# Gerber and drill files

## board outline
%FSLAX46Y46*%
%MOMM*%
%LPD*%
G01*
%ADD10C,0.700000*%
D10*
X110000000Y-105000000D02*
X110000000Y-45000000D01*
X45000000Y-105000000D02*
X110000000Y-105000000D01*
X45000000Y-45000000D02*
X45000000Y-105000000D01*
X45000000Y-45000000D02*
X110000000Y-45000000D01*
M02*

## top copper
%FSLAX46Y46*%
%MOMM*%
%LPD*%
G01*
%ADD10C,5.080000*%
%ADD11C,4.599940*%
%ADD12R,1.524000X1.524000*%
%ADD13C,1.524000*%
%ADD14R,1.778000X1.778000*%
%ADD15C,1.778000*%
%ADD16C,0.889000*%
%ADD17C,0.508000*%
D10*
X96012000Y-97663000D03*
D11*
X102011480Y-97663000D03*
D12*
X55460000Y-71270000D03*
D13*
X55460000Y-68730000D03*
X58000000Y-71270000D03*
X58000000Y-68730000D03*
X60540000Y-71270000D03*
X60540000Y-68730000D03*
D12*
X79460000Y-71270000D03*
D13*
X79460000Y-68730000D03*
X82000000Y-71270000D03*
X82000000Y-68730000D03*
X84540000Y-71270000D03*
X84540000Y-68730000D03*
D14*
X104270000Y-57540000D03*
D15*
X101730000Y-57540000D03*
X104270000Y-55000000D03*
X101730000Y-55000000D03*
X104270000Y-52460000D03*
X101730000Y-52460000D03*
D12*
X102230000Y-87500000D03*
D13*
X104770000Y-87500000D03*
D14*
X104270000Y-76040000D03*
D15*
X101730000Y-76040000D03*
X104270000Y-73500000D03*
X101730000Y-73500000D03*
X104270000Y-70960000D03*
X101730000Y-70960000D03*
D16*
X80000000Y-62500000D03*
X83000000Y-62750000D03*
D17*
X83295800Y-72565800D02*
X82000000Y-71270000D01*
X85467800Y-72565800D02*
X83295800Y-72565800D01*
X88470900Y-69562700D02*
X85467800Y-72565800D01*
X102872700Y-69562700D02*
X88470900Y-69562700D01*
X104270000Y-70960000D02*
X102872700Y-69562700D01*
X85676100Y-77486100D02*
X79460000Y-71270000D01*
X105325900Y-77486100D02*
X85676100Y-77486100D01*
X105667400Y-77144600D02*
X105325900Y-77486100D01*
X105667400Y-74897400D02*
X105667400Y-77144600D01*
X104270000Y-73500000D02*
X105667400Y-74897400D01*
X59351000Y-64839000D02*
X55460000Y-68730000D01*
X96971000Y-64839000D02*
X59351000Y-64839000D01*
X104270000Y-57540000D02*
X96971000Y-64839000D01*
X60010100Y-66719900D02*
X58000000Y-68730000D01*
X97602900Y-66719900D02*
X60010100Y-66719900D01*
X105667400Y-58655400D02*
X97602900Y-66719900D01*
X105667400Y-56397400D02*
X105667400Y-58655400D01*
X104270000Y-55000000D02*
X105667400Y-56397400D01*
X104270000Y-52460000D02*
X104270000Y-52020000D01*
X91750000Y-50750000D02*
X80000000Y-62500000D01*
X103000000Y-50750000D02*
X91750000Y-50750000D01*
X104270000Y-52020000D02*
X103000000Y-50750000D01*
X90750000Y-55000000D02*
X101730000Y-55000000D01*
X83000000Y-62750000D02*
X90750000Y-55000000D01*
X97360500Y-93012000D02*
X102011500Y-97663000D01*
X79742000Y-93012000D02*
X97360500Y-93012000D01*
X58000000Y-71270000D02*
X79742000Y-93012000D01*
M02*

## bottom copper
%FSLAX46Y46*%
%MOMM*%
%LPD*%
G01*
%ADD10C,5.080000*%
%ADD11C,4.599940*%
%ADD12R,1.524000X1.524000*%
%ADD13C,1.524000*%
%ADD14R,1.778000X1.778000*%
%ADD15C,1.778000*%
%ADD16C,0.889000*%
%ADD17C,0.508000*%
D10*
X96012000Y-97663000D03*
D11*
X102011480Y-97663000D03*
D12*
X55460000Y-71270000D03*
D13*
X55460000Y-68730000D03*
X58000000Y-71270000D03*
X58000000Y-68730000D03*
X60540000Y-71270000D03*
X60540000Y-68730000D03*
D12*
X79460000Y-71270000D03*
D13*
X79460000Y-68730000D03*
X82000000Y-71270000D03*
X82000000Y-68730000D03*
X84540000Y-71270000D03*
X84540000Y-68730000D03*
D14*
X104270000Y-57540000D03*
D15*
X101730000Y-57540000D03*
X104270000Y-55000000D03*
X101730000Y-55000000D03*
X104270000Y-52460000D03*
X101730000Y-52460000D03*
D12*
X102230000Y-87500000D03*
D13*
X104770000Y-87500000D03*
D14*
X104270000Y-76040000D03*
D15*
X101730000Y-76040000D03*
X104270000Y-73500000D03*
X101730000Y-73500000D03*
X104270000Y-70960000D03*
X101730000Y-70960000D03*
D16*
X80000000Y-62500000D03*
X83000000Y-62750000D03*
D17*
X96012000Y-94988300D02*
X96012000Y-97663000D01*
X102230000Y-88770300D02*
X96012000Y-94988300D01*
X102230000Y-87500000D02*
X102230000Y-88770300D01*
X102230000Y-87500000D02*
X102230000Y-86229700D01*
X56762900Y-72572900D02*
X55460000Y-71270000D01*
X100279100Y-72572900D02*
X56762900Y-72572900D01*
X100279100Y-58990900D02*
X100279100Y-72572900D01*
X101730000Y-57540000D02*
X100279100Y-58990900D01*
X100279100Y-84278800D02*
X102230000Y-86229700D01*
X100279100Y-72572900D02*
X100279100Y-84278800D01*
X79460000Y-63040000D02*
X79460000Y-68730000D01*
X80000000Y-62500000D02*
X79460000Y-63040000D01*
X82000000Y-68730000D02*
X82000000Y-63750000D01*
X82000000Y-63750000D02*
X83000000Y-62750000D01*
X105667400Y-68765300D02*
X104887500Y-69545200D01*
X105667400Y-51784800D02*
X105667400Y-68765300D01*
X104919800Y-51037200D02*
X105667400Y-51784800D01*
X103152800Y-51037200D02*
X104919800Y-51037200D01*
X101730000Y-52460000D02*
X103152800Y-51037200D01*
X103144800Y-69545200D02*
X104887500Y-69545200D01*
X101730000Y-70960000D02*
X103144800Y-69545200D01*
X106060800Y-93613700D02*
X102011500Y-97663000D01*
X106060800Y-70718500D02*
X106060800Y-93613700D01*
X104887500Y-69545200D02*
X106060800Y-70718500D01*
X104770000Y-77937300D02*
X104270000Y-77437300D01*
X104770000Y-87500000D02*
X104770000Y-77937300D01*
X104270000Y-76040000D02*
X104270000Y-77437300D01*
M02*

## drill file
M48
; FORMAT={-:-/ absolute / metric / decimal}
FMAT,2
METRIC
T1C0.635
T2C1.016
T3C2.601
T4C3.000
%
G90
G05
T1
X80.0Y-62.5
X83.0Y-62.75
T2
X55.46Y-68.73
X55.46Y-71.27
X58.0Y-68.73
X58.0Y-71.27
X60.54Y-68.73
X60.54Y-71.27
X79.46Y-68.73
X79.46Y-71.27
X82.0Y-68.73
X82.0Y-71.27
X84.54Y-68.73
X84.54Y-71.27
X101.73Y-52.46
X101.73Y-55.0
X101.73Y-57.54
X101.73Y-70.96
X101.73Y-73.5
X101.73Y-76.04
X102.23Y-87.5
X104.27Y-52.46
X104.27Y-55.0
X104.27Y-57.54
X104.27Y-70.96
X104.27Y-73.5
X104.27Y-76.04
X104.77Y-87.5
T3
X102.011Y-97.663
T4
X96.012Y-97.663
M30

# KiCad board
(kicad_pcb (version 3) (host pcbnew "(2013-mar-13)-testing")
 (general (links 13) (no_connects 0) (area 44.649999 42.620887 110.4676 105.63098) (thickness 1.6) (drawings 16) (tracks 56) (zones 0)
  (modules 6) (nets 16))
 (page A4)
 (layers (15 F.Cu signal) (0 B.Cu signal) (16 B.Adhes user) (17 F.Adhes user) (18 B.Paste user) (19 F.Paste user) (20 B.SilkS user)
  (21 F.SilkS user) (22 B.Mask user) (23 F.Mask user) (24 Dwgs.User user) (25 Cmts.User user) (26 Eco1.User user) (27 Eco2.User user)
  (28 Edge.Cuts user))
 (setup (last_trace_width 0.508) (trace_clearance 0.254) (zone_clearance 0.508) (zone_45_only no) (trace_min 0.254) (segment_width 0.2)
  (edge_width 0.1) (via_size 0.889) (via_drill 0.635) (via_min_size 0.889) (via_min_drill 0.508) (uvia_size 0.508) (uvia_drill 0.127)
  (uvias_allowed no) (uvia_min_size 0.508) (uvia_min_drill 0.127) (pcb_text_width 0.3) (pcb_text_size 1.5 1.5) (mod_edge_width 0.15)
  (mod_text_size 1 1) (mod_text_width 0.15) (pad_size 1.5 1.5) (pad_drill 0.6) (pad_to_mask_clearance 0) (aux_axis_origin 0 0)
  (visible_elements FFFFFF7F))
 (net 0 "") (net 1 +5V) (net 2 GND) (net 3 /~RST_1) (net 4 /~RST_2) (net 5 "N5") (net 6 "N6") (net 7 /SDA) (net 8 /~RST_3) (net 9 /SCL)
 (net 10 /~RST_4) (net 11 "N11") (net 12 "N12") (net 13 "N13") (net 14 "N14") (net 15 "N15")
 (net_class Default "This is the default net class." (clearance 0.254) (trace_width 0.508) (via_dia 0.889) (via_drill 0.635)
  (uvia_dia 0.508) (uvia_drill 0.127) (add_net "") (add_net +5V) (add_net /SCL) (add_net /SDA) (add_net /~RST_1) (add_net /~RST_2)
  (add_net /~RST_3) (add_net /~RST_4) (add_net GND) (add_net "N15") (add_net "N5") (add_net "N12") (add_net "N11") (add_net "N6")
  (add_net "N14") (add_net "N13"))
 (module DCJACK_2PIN (layer F.Cu) (at 96.012 97.663)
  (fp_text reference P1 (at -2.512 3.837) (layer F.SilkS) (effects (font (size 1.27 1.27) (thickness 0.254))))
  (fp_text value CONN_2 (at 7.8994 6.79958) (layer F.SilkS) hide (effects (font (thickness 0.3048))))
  (pad 1 thru_hole circle (at 0 0) (size 5.08 5.08) (drill 2.99974) (layers *.Cu *.Mask F.SilkS) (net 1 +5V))
  (pad 2 thru_hole circle (at 5.99948 0) (size 4.59994 4.59994) (drill 2.60096) (layers *.Cu *.Mask F.SilkS) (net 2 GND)))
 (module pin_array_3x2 (layer F.Cu) (at 58 70)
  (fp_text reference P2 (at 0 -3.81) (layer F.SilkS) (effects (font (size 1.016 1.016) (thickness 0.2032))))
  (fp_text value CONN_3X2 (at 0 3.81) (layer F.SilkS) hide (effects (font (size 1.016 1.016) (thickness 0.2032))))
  (pad 1 thru_hole rect (at -2.54 1.27) (size 1.524 1.524) (drill 1.016) (layers *.Cu *.Mask F.SilkS) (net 1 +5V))
  (pad 2 thru_hole circle (at -2.54 -1.27) (size 1.524 1.524) (drill 1.016) (layers *.Cu *.Mask F.SilkS) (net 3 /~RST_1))
  (pad 3 thru_hole circle (at 0 1.27) (size 1.524 1.524) (drill 1.016) (layers *.Cu *.Mask F.SilkS) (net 2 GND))
  (pad 4 thru_hole circle (at 0 -1.27) (size 1.524 1.524) (drill 1.016) (layers *.Cu *.Mask F.SilkS) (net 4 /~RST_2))
  (pad 5 thru_hole circle (at 2.54 1.27) (size 1.524 1.524) (drill 1.016) (layers *.Cu *.Mask F.SilkS) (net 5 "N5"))
  (pad 6 thru_hole circle (at 2.54 -1.27) (size 1.524 1.524) (drill 1.016) (layers *.Cu *.Mask F.SilkS) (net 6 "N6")))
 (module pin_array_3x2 (layer F.Cu) (at 82 70)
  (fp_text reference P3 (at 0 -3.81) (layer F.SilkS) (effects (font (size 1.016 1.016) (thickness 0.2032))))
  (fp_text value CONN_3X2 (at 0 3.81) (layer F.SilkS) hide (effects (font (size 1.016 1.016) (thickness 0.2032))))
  (pad 1 thru_hole rect (at -2.54 1.27) (size 1.524 1.524) (drill 1.016) (layers *.Cu *.Mask F.SilkS) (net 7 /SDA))
  (pad 2 thru_hole circle (at -2.54 -1.27) (size 1.524 1.524) (drill 1.016) (layers *.Cu *.Mask F.SilkS) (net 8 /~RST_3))
  (pad 3 thru_hole circle (at 0 1.27) (size 1.524 1.524) (drill 1.016) (layers *.Cu *.Mask F.SilkS) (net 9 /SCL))
  (pad 4 thru_hole circle (at 0 -1.27) (size 1.524 1.524) (drill 1.016) (layers *.Cu *.Mask F.SilkS) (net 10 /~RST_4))
  (pad 5 thru_hole circle (at 2.54 1.27) (size 1.524 1.524) (drill 1.016) (layers *.Cu *.Mask F.SilkS) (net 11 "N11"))
  (pad 6 thru_hole circle (at 2.54 -1.27) (size 1.524 1.524) (drill 1.016) (layers *.Cu *.Mask F.SilkS) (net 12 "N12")))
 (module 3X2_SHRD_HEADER (layer F.Cu) (at 103 55 90)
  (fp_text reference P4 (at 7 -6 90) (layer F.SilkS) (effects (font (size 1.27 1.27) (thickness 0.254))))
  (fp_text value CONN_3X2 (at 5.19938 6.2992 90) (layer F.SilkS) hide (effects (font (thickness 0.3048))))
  (pad 1 thru_hole rect (at -2.54 1.27 90) (size 1.778 1.778) (drill 1.016) (layers *.Cu *.Mask F.SilkS) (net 3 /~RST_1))
  (pad 2 thru_hole circle (at -2.54 -1.27 90) (size 1.778 1.778) (drill 1.016) (layers *.Cu *.Mask F.SilkS) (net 1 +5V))
  (pad 3 thru_hole circle (at 0 1.27 90) (size 1.778 1.778) (drill 1.016) (layers *.Cu *.Mask F.SilkS) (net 4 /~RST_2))
  (pad 4 thru_hole circle (at 0 -1.27 90) (size 1.778 1.778) (drill 1.016) (layers *.Cu *.Mask F.SilkS) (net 10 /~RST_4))
  (pad 5 thru_hole circle (at 2.54 1.27 90) (size 1.778 1.778) (drill 1.016) (layers *.Cu *.Mask F.SilkS) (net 8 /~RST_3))
  (pad 6 thru_hole circle (at 2.54 -1.27 90) (size 1.778 1.778) (drill 1.016) (layers *.Cu *.Mask F.SilkS) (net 2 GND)))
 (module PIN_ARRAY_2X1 (layer F.Cu) (at 103.5 87.5)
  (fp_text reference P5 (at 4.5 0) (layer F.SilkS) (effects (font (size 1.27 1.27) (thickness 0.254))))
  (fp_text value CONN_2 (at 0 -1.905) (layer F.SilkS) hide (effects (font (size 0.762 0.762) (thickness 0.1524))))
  (pad 1 thru_hole rect (at -1.27 0) (size 1.524 1.524) (drill 1.016) (layers *.Cu *.Mask F.SilkS) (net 1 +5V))
  (pad 2 thru_hole circle (at 1.27 0) (size 1.524 1.524) (drill 1.016) (layers *.Cu *.Mask F.SilkS) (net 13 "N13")))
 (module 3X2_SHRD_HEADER (layer F.Cu) (at 103 73.5 90)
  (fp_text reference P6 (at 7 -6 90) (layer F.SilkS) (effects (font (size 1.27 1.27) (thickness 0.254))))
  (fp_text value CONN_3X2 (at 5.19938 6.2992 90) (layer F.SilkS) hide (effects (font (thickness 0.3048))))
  (pad 1 thru_hole rect (at -2.54 1.27 90) (size 1.778 1.778) (drill 1.016) (layers *.Cu *.Mask F.SilkS) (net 13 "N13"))
  (pad 2 thru_hole circle (at -2.54 -1.27 90) (size 1.778 1.778) (drill 1.016) (layers *.Cu *.Mask F.SilkS) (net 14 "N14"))
  (pad 3 thru_hole circle (at 0 1.27 90) (size 1.778 1.778) (drill 1.016) (layers *.Cu *.Mask F.SilkS) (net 7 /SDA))
  (pad 4 thru_hole circle (at 0 -1.27 90) (size 1.778 1.778) (drill 1.016) (layers *.Cu *.Mask F.SilkS) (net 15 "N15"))
  (pad 5 thru_hole circle (at 2.54 1.27 90) (size 1.778 1.778) (drill 1.016) (layers *.Cu *.Mask F.SilkS) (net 9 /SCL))
  (pad 6 thru_hole circle (at 2.54 -1.27 90) (size 1.778 1.778) (drill 1.016) (layers *.Cu *.Mask F.SilkS) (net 2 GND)))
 (gr_line (start 110 105) (end 110 45) (angle 90) (layer Edge.Cuts) (width 0.7))
 (gr_line (start 45 105) (end 110 105) (angle 90) (layer Edge.Cuts) (width 0.7))
 (gr_line (start 45 45) (end 45 105) (angle 90) (layer Edge.Cuts) (width 0.7))
 (gr_line (start 45 45) (end 110 45) (angle 90) (layer Edge.Cuts) (width 0.7))
 (segment (start 96.012 94.9883) (end 96.012 97.663) (width 0.508) (layer B.Cu) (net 1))
 (segment (start 102.23 88.7703) (end 96.012 94.9883) (width 0.508) (layer B.Cu) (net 1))
 (segment (start 102.23 87.5) (end 102.23 88.7703) (width 0.508) (layer B.Cu) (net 1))
 (segment (start 102.23 87.5) (end 102.23 86.2297) (width 0.508) (layer B.Cu) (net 1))
 (segment (start 56.7629 72.5729) (end 55.46 71.27) (width 0.508) (layer B.Cu) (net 1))
 (segment (start 100.2791 72.5729) (end 56.7629 72.5729) (width 0.508) (layer B.Cu) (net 1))
 (segment (start 100.2791 58.9909) (end 100.2791 72.5729) (width 0.508) (layer B.Cu) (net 1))
 (segment (start 101.73 57.54) (end 100.2791 58.9909) (width 0.508) (layer B.Cu) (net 1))
 (segment (start 100.2791 84.2788) (end 102.23 86.2297) (width 0.508) (layer B.Cu) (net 1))
 (segment (start 100.2791 72.5729) (end 100.2791 84.2788) (width 0.508) (layer B.Cu) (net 1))
 (segment (start 83.2958 72.5658) (end 82 71.27) (width 0.508) (layer F.Cu) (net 9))
 (segment (start 85.4678 72.5658) (end 83.2958 72.5658) (width 0.508) (layer F.Cu) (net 9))
 (segment (start 88.4709 69.5627) (end 85.4678 72.5658) (width 0.508) (layer F.Cu) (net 9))
 (segment (start 102.8727 69.5627) (end 88.4709 69.5627) (width 0.508) (layer F.Cu) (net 9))
 (segment (start 104.27 70.96) (end 102.8727 69.5627) (width 0.508) (layer F.Cu) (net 9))
 (segment (start 85.6761 77.4861) (end 79.46 71.27) (width 0.508) (layer F.Cu) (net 7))
 (segment (start 105.3259 77.4861) (end 85.6761 77.4861) (width 0.508) (layer F.Cu) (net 7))
 (segment (start 105.6674 77.1446) (end 105.3259 77.4861) (width 0.508) (layer F.Cu) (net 7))
 (segment (start 105.6674 74.8974) (end 105.6674 77.1446) (width 0.508) (layer F.Cu) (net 7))
 (segment (start 104.27 73.5) (end 105.6674 74.8974) (width 0.508) (layer F.Cu) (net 7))
 (segment (start 59.351 64.839) (end 55.46 68.73) (width 0.508) (layer F.Cu) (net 3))
 (segment (start 96.971 64.839) (end 59.351 64.839) (width 0.508) (layer F.Cu) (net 3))
 (segment (start 104.27 57.54) (end 96.971 64.839) (width 0.508) (layer F.Cu) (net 3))
 (segment (start 60.0101 66.7199) (end 58 68.73) (width 0.508) (layer F.Cu) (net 4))
 (segment (start 97.6029 66.7199) (end 60.0101 66.7199) (width 0.508) (layer F.Cu) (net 4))
 (segment (start 105.6674 58.6554) (end 97.6029 66.7199) (width 0.508) (layer F.Cu) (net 4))
 (segment (start 105.6674 56.3974) (end 105.6674 58.6554) (width 0.508) (layer F.Cu) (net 4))
 (segment (start 104.27 55) (end 105.6674 56.3974) (width 0.508) (layer F.Cu) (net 4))
 (segment (start 104.27 52.46) (end 104.27 52.02) (width 0.508) (layer F.Cu) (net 8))
 (segment (start 79.46 63.04) (end 79.46 68.73) (width 0.508) (layer B.Cu) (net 8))
 (segment (start 80 62.5) (end 79.46 63.04) (width 0.508) (layer B.Cu) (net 8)) (via (at 80 62.5) (size 0.889) (layers F.Cu B.Cu) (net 8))
 (segment (start 91.75 50.75) (end 80 62.5) (width 0.508) (layer F.Cu) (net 8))
 (segment (start 103 50.75) (end 91.75 50.75) (width 0.508) (layer F.Cu) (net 8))
 (segment (start 104.27 52.02) (end 103 50.75) (width 0.508) (layer F.Cu) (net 8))
 (segment (start 82 68.73) (end 82 63.75) (width 0.508) (layer B.Cu) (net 10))
 (segment (start 90.75 55) (end 101.73 55) (width 0.508) (layer F.Cu) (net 10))
 (segment (start 83 62.75) (end 90.75 55) (width 0.508) (layer F.Cu) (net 10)) (via (at 83 62.75) (size 0.889) (layers F.Cu B.Cu) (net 10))
 (segment (start 82 63.75) (end 83 62.75) (width 0.508) (layer B.Cu) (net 10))
 (segment (start 97.3605 93.012) (end 102.0115 97.663) (width 0.508) (layer F.Cu) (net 2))
 (segment (start 79.742 93.012) (end 97.3605 93.012) (width 0.508) (layer F.Cu) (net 2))
 (segment (start 58 71.27) (end 79.742 93.012) (width 0.508) (layer F.Cu) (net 2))
 (segment (start 105.6674 68.7653) (end 104.8875 69.5452) (width 0.508) (layer B.Cu) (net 2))
 (segment (start 105.6674 51.7848) (end 105.6674 68.7653) (width 0.508) (layer B.Cu) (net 2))
 (segment (start 104.9198 51.0372) (end 105.6674 51.7848) (width 0.508) (layer B.Cu) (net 2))
 (segment (start 103.1528 51.0372) (end 104.9198 51.0372) (width 0.508) (layer B.Cu) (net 2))
 (segment (start 101.73 52.46) (end 103.1528 51.0372) (width 0.508) (layer B.Cu) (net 2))
 (segment (start 103.1448 69.5452) (end 104.8875 69.5452) (width 0.508) (layer B.Cu) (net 2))
 (segment (start 101.73 70.96) (end 103.1448 69.5452) (width 0.508) (layer B.Cu) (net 2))
 (segment (start 106.0608 93.6137) (end 102.0115 97.663) (width 0.508) (layer B.Cu) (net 2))
 (segment (start 106.0608 70.7185) (end 106.0608 93.6137) (width 0.508) (layer B.Cu) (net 2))
 (segment (start 104.8875 69.5452) (end 106.0608 70.7185) (width 0.508) (layer B.Cu) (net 2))
 (segment (start 104.77 77.9373) (end 104.27 77.4373) (width 0.508) (layer B.Cu) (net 13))
 (segment (start 104.77 87.5) (end 104.77 77.9373) (width 0.508) (layer B.Cu) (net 13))
 (segment (start 104.27 76.04) (end 104.27 77.4373) (width 0.508) (layer B.Cu) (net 13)))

